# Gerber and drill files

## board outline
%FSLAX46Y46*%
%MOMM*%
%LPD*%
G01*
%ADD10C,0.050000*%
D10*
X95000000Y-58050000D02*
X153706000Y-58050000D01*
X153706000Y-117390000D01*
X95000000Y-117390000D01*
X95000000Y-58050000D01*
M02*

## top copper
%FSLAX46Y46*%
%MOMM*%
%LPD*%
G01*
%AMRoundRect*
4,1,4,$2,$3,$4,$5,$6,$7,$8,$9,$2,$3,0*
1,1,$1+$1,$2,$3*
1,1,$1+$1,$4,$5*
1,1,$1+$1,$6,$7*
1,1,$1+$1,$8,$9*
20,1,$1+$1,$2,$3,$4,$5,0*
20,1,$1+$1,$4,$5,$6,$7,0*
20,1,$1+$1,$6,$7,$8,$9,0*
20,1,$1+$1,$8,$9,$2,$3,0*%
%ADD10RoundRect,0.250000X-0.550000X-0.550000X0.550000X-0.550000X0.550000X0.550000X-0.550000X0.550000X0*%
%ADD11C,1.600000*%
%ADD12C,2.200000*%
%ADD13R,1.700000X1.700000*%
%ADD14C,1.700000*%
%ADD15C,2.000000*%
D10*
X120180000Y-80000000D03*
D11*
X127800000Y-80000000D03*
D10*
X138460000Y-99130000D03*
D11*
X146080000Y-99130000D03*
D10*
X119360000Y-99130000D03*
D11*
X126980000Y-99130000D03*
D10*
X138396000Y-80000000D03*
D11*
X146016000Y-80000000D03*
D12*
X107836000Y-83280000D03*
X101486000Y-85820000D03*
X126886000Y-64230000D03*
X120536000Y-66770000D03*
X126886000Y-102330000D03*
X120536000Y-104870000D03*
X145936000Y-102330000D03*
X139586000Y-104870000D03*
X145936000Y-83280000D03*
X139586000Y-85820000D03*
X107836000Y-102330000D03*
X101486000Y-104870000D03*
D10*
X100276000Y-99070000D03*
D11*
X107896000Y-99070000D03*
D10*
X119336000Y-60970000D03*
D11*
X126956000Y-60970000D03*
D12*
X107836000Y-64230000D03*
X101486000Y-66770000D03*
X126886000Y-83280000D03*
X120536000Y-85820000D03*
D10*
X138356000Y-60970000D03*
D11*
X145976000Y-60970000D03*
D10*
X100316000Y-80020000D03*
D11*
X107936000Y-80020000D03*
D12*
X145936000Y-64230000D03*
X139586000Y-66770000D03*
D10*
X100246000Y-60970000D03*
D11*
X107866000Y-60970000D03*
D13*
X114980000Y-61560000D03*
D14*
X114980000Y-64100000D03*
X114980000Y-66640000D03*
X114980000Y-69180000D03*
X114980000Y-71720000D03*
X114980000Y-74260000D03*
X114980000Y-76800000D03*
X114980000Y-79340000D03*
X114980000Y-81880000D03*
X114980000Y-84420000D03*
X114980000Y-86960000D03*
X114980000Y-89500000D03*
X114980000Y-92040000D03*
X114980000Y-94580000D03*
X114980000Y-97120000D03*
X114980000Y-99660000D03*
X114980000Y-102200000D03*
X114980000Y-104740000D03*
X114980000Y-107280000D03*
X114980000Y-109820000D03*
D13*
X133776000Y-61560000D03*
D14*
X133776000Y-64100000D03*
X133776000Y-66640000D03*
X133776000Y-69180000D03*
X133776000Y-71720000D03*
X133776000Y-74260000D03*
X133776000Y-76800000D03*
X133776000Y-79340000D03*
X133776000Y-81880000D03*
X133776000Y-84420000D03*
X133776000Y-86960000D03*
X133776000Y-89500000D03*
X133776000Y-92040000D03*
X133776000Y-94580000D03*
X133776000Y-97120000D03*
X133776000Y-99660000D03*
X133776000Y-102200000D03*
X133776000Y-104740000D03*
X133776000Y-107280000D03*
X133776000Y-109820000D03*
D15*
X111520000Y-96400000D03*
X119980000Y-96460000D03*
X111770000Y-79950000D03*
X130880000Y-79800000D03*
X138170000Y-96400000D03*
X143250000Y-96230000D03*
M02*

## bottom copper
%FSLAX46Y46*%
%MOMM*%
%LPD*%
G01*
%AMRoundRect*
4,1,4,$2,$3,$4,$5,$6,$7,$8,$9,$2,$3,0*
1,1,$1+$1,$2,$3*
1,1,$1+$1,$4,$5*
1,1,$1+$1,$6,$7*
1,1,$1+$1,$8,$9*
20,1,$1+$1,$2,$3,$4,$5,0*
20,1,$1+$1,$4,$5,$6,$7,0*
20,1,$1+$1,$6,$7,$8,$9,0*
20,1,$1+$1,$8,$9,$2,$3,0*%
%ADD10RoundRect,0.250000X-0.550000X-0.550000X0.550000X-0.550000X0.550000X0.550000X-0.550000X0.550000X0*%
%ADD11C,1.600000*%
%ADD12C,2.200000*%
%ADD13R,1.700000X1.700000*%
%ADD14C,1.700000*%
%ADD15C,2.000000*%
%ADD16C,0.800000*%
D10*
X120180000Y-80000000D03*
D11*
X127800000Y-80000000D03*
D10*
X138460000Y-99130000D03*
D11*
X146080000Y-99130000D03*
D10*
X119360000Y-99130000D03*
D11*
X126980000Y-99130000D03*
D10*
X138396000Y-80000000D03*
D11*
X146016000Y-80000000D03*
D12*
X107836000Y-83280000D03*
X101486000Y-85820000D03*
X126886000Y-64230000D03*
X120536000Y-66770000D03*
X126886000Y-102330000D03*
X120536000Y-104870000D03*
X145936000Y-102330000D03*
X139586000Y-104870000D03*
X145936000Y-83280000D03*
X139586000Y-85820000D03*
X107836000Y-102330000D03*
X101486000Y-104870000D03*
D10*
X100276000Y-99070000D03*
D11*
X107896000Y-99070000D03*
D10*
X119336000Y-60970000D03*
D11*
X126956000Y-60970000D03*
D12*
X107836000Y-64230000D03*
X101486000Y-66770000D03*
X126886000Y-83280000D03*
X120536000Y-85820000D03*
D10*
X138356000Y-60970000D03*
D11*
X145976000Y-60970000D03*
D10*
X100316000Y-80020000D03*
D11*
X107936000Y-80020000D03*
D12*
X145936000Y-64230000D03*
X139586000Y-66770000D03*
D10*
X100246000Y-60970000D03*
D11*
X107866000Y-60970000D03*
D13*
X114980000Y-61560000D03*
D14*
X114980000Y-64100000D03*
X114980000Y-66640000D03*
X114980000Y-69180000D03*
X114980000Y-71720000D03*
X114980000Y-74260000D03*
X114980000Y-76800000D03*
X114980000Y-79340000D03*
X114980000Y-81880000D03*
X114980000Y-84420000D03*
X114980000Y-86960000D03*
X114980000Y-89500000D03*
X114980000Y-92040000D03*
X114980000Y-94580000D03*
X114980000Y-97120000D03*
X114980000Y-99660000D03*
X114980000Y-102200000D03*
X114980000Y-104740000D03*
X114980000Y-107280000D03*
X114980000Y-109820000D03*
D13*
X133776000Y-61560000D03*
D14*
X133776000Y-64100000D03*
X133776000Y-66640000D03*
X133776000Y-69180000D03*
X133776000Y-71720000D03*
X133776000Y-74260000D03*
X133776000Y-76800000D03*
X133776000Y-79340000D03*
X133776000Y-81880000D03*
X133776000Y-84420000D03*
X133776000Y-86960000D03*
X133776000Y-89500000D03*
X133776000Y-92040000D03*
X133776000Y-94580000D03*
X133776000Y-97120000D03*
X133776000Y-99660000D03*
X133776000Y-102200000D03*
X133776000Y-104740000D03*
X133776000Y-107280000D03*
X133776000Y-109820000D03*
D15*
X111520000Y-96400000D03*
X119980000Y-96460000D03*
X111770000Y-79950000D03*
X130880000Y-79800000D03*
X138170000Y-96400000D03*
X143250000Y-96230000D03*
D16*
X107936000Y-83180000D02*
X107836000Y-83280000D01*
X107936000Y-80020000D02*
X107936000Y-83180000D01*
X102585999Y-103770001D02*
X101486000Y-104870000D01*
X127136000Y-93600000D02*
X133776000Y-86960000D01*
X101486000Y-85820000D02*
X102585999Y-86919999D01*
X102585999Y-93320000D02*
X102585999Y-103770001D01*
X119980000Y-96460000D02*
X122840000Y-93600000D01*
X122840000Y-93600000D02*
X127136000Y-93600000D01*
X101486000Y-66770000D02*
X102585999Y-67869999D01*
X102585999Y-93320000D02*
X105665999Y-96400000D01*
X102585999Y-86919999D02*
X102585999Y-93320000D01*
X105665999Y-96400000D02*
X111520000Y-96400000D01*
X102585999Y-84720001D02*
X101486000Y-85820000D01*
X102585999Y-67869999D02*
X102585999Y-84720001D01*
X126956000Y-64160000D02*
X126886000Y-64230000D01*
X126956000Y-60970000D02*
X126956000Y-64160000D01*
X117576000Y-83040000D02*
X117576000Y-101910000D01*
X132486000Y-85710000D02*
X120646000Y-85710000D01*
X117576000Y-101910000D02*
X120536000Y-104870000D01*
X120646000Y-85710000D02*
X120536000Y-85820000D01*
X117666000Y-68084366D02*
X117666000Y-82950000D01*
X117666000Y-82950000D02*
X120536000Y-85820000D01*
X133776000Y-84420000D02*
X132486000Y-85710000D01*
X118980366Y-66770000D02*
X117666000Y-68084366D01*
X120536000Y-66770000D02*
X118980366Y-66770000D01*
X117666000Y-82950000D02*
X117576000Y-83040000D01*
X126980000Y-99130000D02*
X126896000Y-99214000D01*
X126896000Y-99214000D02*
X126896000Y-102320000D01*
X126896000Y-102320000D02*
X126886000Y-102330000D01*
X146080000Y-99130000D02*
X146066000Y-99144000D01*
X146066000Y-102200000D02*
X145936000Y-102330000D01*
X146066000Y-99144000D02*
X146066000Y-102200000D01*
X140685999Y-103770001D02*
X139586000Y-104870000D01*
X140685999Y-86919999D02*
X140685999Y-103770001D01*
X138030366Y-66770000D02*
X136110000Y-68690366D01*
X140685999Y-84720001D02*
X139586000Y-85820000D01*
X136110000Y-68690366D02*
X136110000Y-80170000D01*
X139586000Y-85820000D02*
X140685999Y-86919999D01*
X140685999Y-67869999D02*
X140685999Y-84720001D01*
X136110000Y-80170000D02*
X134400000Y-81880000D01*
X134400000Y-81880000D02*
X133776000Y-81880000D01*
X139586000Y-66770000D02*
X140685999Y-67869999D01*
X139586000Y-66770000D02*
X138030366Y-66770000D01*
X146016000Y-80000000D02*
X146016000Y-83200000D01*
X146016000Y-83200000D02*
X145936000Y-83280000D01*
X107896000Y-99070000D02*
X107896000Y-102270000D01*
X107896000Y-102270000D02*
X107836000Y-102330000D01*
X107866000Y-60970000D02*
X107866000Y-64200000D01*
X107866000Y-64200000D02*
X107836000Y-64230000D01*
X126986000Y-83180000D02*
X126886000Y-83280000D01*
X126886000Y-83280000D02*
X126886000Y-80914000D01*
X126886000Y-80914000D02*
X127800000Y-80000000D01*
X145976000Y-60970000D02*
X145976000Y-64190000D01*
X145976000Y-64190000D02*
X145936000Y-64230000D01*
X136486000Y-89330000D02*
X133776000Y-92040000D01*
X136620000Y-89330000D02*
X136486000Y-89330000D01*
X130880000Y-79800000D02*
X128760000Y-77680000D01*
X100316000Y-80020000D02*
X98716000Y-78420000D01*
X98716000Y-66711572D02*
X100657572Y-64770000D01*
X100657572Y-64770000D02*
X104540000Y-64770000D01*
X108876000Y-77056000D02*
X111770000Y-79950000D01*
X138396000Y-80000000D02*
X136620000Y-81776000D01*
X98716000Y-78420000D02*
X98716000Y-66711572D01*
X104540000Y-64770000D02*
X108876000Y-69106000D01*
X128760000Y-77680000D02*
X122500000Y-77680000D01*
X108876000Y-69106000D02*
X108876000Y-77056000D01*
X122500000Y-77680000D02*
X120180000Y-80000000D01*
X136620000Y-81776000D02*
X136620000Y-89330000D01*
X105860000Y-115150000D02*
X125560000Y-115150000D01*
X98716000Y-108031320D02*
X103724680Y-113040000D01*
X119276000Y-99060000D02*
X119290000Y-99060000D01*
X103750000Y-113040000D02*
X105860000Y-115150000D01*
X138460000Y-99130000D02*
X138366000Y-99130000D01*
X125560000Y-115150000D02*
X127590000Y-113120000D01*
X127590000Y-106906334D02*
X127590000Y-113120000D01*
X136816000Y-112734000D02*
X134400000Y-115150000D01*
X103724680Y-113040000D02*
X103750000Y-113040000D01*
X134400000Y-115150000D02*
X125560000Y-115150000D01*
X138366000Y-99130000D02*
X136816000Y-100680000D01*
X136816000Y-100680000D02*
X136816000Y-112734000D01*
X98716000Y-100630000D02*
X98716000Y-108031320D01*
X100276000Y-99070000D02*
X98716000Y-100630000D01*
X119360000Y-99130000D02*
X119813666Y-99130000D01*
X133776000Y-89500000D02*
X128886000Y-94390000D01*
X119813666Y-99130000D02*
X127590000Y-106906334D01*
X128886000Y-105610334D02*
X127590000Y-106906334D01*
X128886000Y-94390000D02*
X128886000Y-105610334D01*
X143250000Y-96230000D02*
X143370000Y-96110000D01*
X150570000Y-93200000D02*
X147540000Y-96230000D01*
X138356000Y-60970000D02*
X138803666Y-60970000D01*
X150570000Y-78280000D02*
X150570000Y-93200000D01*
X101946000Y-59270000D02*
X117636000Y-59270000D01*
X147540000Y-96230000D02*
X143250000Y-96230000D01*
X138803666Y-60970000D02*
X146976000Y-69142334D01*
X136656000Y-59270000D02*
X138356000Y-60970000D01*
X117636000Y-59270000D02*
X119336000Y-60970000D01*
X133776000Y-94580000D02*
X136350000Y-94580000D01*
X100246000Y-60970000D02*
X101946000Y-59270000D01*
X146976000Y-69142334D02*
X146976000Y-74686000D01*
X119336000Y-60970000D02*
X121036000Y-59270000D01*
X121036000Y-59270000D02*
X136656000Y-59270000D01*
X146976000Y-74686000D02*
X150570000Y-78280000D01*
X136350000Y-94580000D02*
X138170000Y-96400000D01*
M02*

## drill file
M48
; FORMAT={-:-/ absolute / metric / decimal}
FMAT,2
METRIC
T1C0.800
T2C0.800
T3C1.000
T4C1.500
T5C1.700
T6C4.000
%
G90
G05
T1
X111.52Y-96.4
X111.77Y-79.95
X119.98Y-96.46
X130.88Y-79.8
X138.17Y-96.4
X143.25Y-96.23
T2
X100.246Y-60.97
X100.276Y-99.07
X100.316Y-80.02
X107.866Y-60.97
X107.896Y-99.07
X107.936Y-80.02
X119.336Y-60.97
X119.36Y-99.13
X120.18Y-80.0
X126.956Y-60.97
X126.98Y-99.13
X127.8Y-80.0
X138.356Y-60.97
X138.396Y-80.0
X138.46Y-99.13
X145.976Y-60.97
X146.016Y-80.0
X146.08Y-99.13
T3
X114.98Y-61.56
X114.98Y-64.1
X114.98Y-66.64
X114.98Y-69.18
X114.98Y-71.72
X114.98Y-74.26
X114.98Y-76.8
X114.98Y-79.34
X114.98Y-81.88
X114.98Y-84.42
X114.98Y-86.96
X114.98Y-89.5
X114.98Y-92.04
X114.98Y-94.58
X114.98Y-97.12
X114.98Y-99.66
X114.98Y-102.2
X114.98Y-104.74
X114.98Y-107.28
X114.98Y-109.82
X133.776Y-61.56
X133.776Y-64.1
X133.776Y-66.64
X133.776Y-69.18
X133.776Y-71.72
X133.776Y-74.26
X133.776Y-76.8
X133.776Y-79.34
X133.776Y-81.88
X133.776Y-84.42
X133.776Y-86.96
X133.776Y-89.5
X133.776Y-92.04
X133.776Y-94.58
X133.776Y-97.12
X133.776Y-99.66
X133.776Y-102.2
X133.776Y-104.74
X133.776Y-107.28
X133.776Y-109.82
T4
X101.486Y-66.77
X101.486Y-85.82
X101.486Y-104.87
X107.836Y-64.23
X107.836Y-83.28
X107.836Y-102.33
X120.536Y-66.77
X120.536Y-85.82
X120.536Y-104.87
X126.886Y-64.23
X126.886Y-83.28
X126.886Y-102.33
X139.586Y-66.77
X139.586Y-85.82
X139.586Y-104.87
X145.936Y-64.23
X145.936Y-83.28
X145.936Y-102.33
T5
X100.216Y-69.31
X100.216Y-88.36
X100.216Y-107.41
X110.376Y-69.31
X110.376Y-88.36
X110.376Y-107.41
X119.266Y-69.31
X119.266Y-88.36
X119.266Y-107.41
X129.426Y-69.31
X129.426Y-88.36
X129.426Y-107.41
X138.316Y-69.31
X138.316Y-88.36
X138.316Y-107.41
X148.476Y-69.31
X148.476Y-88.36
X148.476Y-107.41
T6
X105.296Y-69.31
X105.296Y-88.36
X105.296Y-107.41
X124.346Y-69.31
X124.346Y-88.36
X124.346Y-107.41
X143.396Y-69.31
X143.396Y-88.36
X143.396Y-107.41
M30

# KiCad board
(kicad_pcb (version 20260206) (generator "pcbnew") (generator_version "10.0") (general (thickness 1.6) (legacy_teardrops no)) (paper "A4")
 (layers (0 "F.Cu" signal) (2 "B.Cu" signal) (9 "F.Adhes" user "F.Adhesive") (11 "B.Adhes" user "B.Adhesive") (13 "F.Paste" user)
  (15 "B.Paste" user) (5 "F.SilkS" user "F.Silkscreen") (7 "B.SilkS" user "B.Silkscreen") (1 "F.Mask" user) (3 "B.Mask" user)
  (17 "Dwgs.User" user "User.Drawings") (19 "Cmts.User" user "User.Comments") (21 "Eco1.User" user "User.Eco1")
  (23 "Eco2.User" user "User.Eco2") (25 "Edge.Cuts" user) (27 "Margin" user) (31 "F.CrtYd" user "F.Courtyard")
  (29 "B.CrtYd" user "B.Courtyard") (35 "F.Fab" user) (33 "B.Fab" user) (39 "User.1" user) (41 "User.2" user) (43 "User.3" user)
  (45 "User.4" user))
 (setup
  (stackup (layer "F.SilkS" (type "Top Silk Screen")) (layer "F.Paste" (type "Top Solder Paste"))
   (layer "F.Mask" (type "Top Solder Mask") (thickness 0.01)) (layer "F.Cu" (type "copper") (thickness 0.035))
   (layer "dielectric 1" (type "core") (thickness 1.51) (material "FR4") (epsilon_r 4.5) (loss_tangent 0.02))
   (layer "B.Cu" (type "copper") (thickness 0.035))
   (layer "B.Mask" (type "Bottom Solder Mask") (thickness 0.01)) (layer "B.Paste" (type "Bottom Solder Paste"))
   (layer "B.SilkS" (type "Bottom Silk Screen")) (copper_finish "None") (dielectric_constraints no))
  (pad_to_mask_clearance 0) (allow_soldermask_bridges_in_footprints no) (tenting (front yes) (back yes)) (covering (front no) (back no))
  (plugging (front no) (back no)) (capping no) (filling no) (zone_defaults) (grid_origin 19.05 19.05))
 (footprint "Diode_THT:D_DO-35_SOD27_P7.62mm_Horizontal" (layer "F.Cu") (at 120.18 80)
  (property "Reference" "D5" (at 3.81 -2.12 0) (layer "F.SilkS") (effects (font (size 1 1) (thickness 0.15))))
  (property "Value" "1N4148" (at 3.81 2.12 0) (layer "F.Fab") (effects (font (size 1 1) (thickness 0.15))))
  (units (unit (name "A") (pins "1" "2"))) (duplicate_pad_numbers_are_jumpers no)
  (pad "1" thru_hole roundrect (at 0 0) (size 1.6 1.6) (drill 0.8) (layers "*.Cu" "*.Mask") (remove_unused_layers no)
   (roundrect_rratio 0.15625) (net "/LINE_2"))
  (pad "2" thru_hole circle (at 7.62 0) (size 1.6 1.6) (drill 0.8) (layers "*.Cu" "*.Mask") (remove_unused_layers no) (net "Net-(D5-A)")))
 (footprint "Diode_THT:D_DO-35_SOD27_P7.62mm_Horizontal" (layer "F.Cu") (at 138.46 99.13)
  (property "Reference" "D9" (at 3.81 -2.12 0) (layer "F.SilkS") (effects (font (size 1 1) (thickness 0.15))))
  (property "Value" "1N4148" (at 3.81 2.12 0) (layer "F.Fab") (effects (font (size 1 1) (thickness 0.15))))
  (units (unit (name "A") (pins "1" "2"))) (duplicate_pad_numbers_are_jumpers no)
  (pad "1" thru_hole roundrect (at 0 0) (size 1.6 1.6) (drill 0.8) (layers "*.Cu" "*.Mask") (remove_unused_layers no)
   (roundrect_rratio 0.15625) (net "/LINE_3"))
  (pad "2" thru_hole circle (at 7.62 0) (size 1.6 1.6) (drill 0.8) (layers "*.Cu" "*.Mask") (remove_unused_layers no) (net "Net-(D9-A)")))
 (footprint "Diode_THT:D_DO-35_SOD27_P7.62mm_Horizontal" (layer "F.Cu") (at 119.36 99.13)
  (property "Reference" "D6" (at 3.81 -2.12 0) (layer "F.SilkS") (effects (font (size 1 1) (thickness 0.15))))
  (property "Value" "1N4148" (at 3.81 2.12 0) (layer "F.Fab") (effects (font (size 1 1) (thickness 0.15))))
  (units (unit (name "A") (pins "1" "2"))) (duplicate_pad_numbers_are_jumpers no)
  (pad "1" thru_hole roundrect (at 0 0) (size 1.6 1.6) (drill 0.8) (layers "*.Cu" "*.Mask") (remove_unused_layers no)
   (roundrect_rratio 0.15625) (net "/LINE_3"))
  (pad "2" thru_hole circle (at 7.62 0) (size 1.6 1.6) (drill 0.8) (layers "*.Cu" "*.Mask") (remove_unused_layers no) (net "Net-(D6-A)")))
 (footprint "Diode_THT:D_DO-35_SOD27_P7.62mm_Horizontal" (layer "F.Cu") (at 138.396 80)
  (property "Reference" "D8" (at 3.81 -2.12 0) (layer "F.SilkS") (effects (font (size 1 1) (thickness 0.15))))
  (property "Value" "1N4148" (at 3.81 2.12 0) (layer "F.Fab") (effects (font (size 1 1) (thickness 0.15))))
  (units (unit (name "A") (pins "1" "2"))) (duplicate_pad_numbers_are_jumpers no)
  (pad "1" thru_hole roundrect (at 0 0) (size 1.6 1.6) (drill 0.8) (layers "*.Cu" "*.Mask") (remove_unused_layers no)
   (roundrect_rratio 0.15625) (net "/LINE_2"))
  (pad "2" thru_hole circle (at 7.62 0) (size 1.6 1.6) (drill 0.8) (layers "*.Cu" "*.Mask") (remove_unused_layers no) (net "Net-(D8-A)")))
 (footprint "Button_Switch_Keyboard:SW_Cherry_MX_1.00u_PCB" (layer "F.Cu") (at 107.836 83.28)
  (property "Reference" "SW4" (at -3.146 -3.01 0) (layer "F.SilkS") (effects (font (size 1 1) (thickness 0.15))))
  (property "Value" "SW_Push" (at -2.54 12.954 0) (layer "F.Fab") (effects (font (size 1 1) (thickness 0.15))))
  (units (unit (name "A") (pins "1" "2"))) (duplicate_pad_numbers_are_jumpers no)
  (pad "" np_thru_hole circle (at -7.62 5.08) (size 1.7 1.7) (drill 1.7) (layers "*.Cu" "*.Mask"))
  (pad "" np_thru_hole circle (at -2.54 5.08) (size 4 4) (drill 4) (layers "*.Cu" "*.Mask"))
  (pad "" np_thru_hole circle (at 2.54 5.08) (size 1.7 1.7) (drill 1.7) (layers "*.Cu" "*.Mask"))
  (pad "1" thru_hole circle (at 0 0) (size 2.2 2.2) (drill 1.5) (layers "*.Cu" "*.Mask") (remove_unused_layers no) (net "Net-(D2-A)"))
  (pad "2" thru_hole circle (at -6.35 2.54) (size 2.2 2.2) (drill 1.5) (layers "*.Cu" "*.Mask") (remove_unused_layers no) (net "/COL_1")))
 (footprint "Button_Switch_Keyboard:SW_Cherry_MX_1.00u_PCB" (layer "F.Cu") (at 126.886 64.23)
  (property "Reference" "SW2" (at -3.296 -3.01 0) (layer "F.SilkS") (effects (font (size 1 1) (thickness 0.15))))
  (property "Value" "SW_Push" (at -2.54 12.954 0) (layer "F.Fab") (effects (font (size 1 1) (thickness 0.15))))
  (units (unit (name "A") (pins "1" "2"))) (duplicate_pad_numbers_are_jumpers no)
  (pad "" np_thru_hole circle (at -7.62 5.08) (size 1.7 1.7) (drill 1.7) (layers "*.Cu" "*.Mask"))
  (pad "" np_thru_hole circle (at -2.54 5.08) (size 4 4) (drill 4) (layers "*.Cu" "*.Mask"))
  (pad "" np_thru_hole circle (at 2.54 5.08) (size 1.7 1.7) (drill 1.7) (layers "*.Cu" "*.Mask"))
  (pad "1" thru_hole circle (at 0 0) (size 2.2 2.2) (drill 1.5) (layers "*.Cu" "*.Mask") (remove_unused_layers no) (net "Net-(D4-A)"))
  (pad "2" thru_hole circle (at -6.35 2.54) (size 2.2 2.2) (drill 1.5) (layers "*.Cu" "*.Mask") (remove_unused_layers no) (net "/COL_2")))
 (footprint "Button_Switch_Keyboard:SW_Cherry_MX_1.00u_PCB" (layer "F.Cu") (at 126.886 102.33)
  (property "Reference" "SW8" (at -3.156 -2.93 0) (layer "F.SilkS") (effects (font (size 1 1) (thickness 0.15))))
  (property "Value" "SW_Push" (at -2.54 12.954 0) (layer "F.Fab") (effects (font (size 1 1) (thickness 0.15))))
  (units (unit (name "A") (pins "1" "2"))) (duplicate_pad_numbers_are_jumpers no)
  (pad "" np_thru_hole circle (at -7.62 5.08) (size 1.7 1.7) (drill 1.7) (layers "*.Cu" "*.Mask"))
  (pad "" np_thru_hole circle (at -2.54 5.08) (size 4 4) (drill 4) (layers "*.Cu" "*.Mask"))
  (pad "" np_thru_hole circle (at 2.54 5.08) (size 1.7 1.7) (drill 1.7) (layers "*.Cu" "*.Mask"))
  (pad "1" thru_hole circle (at 0 0) (size 2.2 2.2) (drill 1.5) (layers "*.Cu" "*.Mask") (remove_unused_layers no) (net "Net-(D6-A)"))
  (pad "2" thru_hole circle (at -6.35 2.54) (size 2.2 2.2) (drill 1.5) (layers "*.Cu" "*.Mask") (remove_unused_layers no) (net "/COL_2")))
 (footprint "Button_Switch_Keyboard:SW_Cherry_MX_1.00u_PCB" (layer "F.Cu") (at 145.936 102.33)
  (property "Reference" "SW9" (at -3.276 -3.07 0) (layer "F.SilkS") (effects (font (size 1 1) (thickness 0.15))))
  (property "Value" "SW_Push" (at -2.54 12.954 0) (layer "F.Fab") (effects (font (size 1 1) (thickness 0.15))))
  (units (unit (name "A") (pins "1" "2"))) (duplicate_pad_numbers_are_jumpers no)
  (pad "" np_thru_hole circle (at -7.62 5.08) (size 1.7 1.7) (drill 1.7) (layers "*.Cu" "*.Mask"))
  (pad "" np_thru_hole circle (at -2.54 5.08) (size 4 4) (drill 4) (layers "*.Cu" "*.Mask"))
  (pad "" np_thru_hole circle (at 2.54 5.08) (size 1.7 1.7) (drill 1.7) (layers "*.Cu" "*.Mask"))
  (pad "1" thru_hole circle (at 0 0) (size 2.2 2.2) (drill 1.5) (layers "*.Cu" "*.Mask") (remove_unused_layers no) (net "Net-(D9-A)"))
  (pad "2" thru_hole circle (at -6.35 2.54) (size 2.2 2.2) (drill 1.5) (layers "*.Cu" "*.Mask") (remove_unused_layers no) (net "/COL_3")))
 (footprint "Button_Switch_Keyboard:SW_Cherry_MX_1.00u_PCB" (layer "F.Cu") (at 145.936 83.28)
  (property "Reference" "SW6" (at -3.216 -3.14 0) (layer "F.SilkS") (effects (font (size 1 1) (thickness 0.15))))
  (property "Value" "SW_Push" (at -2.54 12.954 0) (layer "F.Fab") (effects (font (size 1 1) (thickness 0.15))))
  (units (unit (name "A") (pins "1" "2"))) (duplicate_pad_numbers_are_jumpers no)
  (pad "" np_thru_hole circle (at -7.62 5.08) (size 1.7 1.7) (drill 1.7) (layers "*.Cu" "*.Mask"))
  (pad "" np_thru_hole circle (at -2.54 5.08) (size 4 4) (drill 4) (layers "*.Cu" "*.Mask"))
  (pad "" np_thru_hole circle (at 2.54 5.08) (size 1.7 1.7) (drill 1.7) (layers "*.Cu" "*.Mask"))
  (pad "1" thru_hole circle (at 0 0) (size 2.2 2.2) (drill 1.5) (layers "*.Cu" "*.Mask") (remove_unused_layers no) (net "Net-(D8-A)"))
  (pad "2" thru_hole circle (at -6.35 2.54) (size 2.2 2.2) (drill 1.5) (layers "*.Cu" "*.Mask") (remove_unused_layers no) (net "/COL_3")))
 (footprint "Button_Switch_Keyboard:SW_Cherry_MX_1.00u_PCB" (layer "F.Cu") (at 107.836 102.33)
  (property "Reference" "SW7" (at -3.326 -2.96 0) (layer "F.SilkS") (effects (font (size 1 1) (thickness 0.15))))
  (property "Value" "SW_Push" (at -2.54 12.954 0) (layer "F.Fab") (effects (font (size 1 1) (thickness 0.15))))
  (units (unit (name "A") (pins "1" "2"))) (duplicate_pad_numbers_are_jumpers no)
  (pad "" np_thru_hole circle (at -7.62 5.08) (size 1.7 1.7) (drill 1.7) (layers "*.Cu" "*.Mask"))
  (pad "" np_thru_hole circle (at -2.54 5.08) (size 4 4) (drill 4) (layers "*.Cu" "*.Mask"))
  (pad "" np_thru_hole circle (at 2.54 5.08) (size 1.7 1.7) (drill 1.7) (layers "*.Cu" "*.Mask"))
  (pad "1" thru_hole circle (at 0 0) (size 2.2 2.2) (drill 1.5) (layers "*.Cu" "*.Mask") (remove_unused_layers no) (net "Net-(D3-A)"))
  (pad "2" thru_hole circle (at -6.35 2.54) (size 2.2 2.2) (drill 1.5) (layers "*.Cu" "*.Mask") (remove_unused_layers no) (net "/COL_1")))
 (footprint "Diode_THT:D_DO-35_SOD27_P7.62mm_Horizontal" (layer "F.Cu") (at 100.276 99.07)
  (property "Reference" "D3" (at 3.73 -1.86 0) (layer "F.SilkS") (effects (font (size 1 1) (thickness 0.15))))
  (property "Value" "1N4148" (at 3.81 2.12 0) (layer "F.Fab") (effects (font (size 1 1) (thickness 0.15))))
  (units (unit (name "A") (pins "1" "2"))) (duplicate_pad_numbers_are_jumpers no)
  (pad "1" thru_hole roundrect (at 0 0) (size 1.6 1.6) (drill 0.8) (layers "*.Cu" "*.Mask") (remove_unused_layers no)
   (roundrect_rratio 0.15625) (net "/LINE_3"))
  (pad "2" thru_hole circle (at 7.62 0) (size 1.6 1.6) (drill 0.8) (layers "*.Cu" "*.Mask") (remove_unused_layers no) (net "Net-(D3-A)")))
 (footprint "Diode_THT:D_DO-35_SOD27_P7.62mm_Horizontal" (layer "F.Cu") (at 119.336 60.97)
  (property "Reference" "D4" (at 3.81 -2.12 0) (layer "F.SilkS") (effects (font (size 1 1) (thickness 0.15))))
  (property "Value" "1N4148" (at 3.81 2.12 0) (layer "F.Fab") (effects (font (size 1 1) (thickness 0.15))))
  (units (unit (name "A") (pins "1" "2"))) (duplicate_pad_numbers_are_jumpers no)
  (pad "1" thru_hole roundrect (at 0 0) (size 1.6 1.6) (drill 0.8) (layers "*.Cu" "*.Mask") (remove_unused_layers no)
   (roundrect_rratio 0.15625) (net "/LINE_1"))
  (pad "2" thru_hole circle (at 7.62 0) (size 1.6 1.6) (drill 0.8) (layers "*.Cu" "*.Mask") (remove_unused_layers no) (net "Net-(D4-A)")))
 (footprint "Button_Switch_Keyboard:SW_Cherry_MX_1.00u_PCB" (layer "F.Cu") (at 107.836 64.23)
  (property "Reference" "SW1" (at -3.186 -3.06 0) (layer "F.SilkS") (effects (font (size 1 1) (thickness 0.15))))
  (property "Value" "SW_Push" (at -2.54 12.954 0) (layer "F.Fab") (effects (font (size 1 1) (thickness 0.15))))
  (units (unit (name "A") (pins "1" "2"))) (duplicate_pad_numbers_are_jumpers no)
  (pad "" np_thru_hole circle (at -7.62 5.08) (size 1.7 1.7) (drill 1.7) (layers "*.Cu" "*.Mask"))
  (pad "" np_thru_hole circle (at -2.54 5.08) (size 4 4) (drill 4) (layers "*.Cu" "*.Mask"))
  (pad "" np_thru_hole circle (at 2.54 5.08) (size 1.7 1.7) (drill 1.7) (layers "*.Cu" "*.Mask"))
  (pad "1" thru_hole circle (at 0 0) (size 2.2 2.2) (drill 1.5) (layers "*.Cu" "*.Mask") (remove_unused_layers no) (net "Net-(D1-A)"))
  (pad "2" thru_hole circle (at -6.35 2.54) (size 2.2 2.2) (drill 1.5) (layers "*.Cu" "*.Mask") (remove_unused_layers no) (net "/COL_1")))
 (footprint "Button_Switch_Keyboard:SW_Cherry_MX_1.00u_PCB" (layer "F.Cu") (at 126.886 83.28)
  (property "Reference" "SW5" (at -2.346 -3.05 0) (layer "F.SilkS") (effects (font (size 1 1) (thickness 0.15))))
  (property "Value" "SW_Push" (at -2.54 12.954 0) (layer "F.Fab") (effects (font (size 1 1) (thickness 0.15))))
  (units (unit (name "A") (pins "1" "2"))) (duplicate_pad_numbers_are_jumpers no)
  (pad "" np_thru_hole circle (at -7.62 5.08) (size 1.7 1.7) (drill 1.7) (layers "*.Cu" "*.Mask"))
  (pad "" np_thru_hole circle (at -2.54 5.08) (size 4 4) (drill 4) (layers "*.Cu" "*.Mask"))
  (pad "" np_thru_hole circle (at 2.54 5.08) (size 1.7 1.7) (drill 1.7) (layers "*.Cu" "*.Mask"))
  (pad "1" thru_hole circle (at 0 0) (size 2.2 2.2) (drill 1.5) (layers "*.Cu" "*.Mask") (remove_unused_layers no) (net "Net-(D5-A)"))
  (pad "2" thru_hole circle (at -6.35 2.54) (size 2.2 2.2) (drill 1.5) (layers "*.Cu" "*.Mask") (remove_unused_layers no) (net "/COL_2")))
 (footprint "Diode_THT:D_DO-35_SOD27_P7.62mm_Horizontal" (layer "F.Cu") (at 138.356 60.97)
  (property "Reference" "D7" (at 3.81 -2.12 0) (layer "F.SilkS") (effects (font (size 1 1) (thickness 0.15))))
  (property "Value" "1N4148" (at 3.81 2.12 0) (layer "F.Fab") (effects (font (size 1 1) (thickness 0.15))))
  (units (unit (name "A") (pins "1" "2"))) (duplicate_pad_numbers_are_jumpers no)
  (pad "1" thru_hole roundrect (at 0 0) (size 1.6 1.6) (drill 0.8) (layers "*.Cu" "*.Mask") (remove_unused_layers no)
   (roundrect_rratio 0.15625) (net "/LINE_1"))
  (pad "2" thru_hole circle (at 7.62 0) (size 1.6 1.6) (drill 0.8) (layers "*.Cu" "*.Mask") (remove_unused_layers no) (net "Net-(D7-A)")))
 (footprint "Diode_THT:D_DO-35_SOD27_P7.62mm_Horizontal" (layer "F.Cu") (at 100.316 80.02)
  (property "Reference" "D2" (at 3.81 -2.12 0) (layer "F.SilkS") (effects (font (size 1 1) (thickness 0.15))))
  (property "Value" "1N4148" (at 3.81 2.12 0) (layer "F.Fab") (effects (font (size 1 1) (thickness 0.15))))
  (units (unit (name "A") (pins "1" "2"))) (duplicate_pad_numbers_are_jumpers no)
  (pad "1" thru_hole roundrect (at 0 0) (size 1.6 1.6) (drill 0.8) (layers "*.Cu" "*.Mask") (remove_unused_layers no)
   (roundrect_rratio 0.15625) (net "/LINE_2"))
  (pad "2" thru_hole circle (at 7.62 0) (size 1.6 1.6) (drill 0.8) (layers "*.Cu" "*.Mask") (remove_unused_layers no) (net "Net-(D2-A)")))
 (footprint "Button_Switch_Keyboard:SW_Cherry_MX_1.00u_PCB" (layer "F.Cu") (at 145.936 64.23)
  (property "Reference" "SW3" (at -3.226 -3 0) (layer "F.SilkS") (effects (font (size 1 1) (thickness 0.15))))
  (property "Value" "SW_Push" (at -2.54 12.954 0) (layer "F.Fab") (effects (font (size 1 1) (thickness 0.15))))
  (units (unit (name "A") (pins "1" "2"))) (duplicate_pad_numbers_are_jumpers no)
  (pad "" np_thru_hole circle (at -7.62 5.08) (size 1.7 1.7) (drill 1.7) (layers "*.Cu" "*.Mask"))
  (pad "" np_thru_hole circle (at -2.54 5.08) (size 4 4) (drill 4) (layers "*.Cu" "*.Mask"))
  (pad "" np_thru_hole circle (at 2.54 5.08) (size 1.7 1.7) (drill 1.7) (layers "*.Cu" "*.Mask"))
  (pad "1" thru_hole circle (at 0 0) (size 2.2 2.2) (drill 1.5) (layers "*.Cu" "*.Mask") (remove_unused_layers no) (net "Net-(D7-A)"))
  (pad "2" thru_hole circle (at -6.35 2.54) (size 2.2 2.2) (drill 1.5) (layers "*.Cu" "*.Mask") (remove_unused_layers no) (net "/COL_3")))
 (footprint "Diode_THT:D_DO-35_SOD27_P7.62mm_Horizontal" (layer "F.Cu") (at 100.246 60.97)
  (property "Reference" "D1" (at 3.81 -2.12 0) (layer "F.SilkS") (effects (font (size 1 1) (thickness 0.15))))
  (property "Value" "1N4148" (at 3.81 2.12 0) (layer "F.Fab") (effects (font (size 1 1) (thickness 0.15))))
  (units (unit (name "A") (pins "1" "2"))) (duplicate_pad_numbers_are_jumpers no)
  (pad "1" thru_hole roundrect (at 0 0) (size 1.6 1.6) (drill 0.8) (layers "*.Cu" "*.Mask") (remove_unused_layers no)
   (roundrect_rratio 0.15625) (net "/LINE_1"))
  (pad "2" thru_hole circle (at 7.62 0) (size 1.6 1.6) (drill 0.8) (layers "*.Cu" "*.Mask") (remove_unused_layers no) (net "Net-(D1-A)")))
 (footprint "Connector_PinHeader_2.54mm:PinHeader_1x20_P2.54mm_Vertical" (layer "B.Cu") (at 114.98 61.56 180)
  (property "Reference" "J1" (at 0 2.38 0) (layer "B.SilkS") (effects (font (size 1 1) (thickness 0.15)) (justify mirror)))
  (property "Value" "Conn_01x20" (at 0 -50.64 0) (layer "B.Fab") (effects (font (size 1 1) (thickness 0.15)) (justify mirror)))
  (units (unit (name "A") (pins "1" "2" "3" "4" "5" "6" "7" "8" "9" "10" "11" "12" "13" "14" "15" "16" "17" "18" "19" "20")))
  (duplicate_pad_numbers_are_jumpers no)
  (pad "1" thru_hole rect (at 0 0 180) (size 1.7 1.7) (drill 1) (layers "*.Cu" "*.Mask") (remove_unused_layers no)
   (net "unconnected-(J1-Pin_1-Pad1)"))
  (pad "2" thru_hole circle (at 0 -2.54 180) (size 1.7 1.7) (drill 1) (layers "*.Cu" "*.Mask") (remove_unused_layers no)
   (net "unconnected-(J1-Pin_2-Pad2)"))
  (pad "3" thru_hole circle (at 0 -5.08 180) (size 1.7 1.7) (drill 1) (layers "*.Cu" "*.Mask") (remove_unused_layers no)
   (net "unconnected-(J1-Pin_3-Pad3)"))
  (pad "4" thru_hole circle (at 0 -7.62 180) (size 1.7 1.7) (drill 1) (layers "*.Cu" "*.Mask") (remove_unused_layers no)
   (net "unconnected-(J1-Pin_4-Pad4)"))
  (pad "5" thru_hole circle (at 0 -10.16 180) (size 1.7 1.7) (drill 1) (layers "*.Cu" "*.Mask") (remove_unused_layers no)
   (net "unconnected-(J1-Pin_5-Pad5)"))
  (pad "6" thru_hole circle (at 0 -12.7 180) (size 1.7 1.7) (drill 1) (layers "*.Cu" "*.Mask") (remove_unused_layers no)
   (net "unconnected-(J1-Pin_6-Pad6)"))
  (pad "7" thru_hole circle (at 0 -15.24 180) (size 1.7 1.7) (drill 1) (layers "*.Cu" "*.Mask") (remove_unused_layers no)
   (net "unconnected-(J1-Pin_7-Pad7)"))
  (pad "8" thru_hole circle (at 0 -17.78 180) (size 1.7 1.7) (drill 1) (layers "*.Cu" "*.Mask") (remove_unused_layers no)
   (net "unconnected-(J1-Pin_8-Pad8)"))
  (pad "9" thru_hole circle (at 0 -20.32 180) (size 1.7 1.7) (drill 1) (layers "*.Cu" "*.Mask") (remove_unused_layers no)
   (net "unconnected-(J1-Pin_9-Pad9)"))
  (pad "10" thru_hole circle (at 0 -22.86 180) (size 1.7 1.7) (drill 1) (layers "*.Cu" "*.Mask") (remove_unused_layers no)
   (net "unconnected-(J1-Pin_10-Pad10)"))
  (pad "11" thru_hole circle (at 0 -25.4 180) (size 1.7 1.7) (drill 1) (layers "*.Cu" "*.Mask") (remove_unused_layers no)
   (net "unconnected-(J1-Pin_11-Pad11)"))
  (pad "12" thru_hole circle (at 0 -27.94 180) (size 1.7 1.7) (drill 1) (layers "*.Cu" "*.Mask") (remove_unused_layers no)
   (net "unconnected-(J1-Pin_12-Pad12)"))
  (pad "13" thru_hole circle (at 0 -30.48 180) (size 1.7 1.7) (drill 1) (layers "*.Cu" "*.Mask") (remove_unused_layers no)
   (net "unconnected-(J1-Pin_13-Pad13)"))
  (pad "14" thru_hole circle (at 0 -33.02 180) (size 1.7 1.7) (drill 1) (layers "*.Cu" "*.Mask") (remove_unused_layers no)
   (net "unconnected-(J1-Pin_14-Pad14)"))
  (pad "15" thru_hole circle (at 0 -35.56 180) (size 1.7 1.7) (drill 1) (layers "*.Cu" "*.Mask") (remove_unused_layers no)
   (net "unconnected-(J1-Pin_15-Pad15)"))
  (pad "16" thru_hole circle (at 0 -38.1 180) (size 1.7 1.7) (drill 1) (layers "*.Cu" "*.Mask") (remove_unused_layers no)
   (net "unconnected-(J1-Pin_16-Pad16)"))
  (pad "17" thru_hole circle (at 0 -40.64 180) (size 1.7 1.7) (drill 1) (layers "*.Cu" "*.Mask") (remove_unused_layers no)
   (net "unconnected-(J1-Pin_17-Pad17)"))
  (pad "18" thru_hole circle (at 0 -43.18 180) (size 1.7 1.7) (drill 1) (layers "*.Cu" "*.Mask") (remove_unused_layers no)
   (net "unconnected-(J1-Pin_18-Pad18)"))
  (pad "19" thru_hole circle (at 0 -45.72 180) (size 1.7 1.7) (drill 1) (layers "*.Cu" "*.Mask") (remove_unused_layers no)
   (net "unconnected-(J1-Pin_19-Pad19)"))
  (pad "20" thru_hole circle (at 0 -48.26 180) (size 1.7 1.7) (drill 1) (layers "*.Cu" "*.Mask") (remove_unused_layers no)
   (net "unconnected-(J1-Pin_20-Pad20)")))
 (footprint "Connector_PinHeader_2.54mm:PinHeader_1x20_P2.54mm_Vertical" (layer "B.Cu") (at 133.776 61.56 180)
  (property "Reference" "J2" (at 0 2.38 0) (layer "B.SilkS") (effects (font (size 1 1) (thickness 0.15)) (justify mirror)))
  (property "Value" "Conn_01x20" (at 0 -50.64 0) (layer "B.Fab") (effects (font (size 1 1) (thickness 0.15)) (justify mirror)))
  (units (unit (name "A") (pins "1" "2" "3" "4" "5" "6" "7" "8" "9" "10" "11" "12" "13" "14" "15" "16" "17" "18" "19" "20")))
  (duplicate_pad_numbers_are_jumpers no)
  (pad "1" thru_hole rect (at 0 0 180) (size 1.7 1.7) (drill 1) (layers "*.Cu" "*.Mask") (remove_unused_layers no)
   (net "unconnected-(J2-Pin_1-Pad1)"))
  (pad "2" thru_hole circle (at 0 -2.54 180) (size 1.7 1.7) (drill 1) (layers "*.Cu" "*.Mask") (remove_unused_layers no)
   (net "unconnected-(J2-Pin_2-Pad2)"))
  (pad "3" thru_hole circle (at 0 -5.08 180) (size 1.7 1.7) (drill 1) (layers "*.Cu" "*.Mask") (remove_unused_layers no)
   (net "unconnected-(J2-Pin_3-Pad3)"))
  (pad "4" thru_hole circle (at 0 -7.62 180) (size 1.7 1.7) (drill 1) (layers "*.Cu" "*.Mask") (remove_unused_layers no)
   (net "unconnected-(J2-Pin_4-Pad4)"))
  (pad "5" thru_hole circle (at 0 -10.16 180) (size 1.7 1.7) (drill 1) (layers "*.Cu" "*.Mask") (remove_unused_layers no)
   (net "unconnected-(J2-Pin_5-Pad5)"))
  (pad "6" thru_hole circle (at 0 -12.7 180) (size 1.7 1.7) (drill 1) (layers "*.Cu" "*.Mask") (remove_unused_layers no)
   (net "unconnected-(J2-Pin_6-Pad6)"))
  (pad "7" thru_hole circle (at 0 -15.24 180) (size 1.7 1.7) (drill 1) (layers "*.Cu" "*.Mask") (remove_unused_layers no)
   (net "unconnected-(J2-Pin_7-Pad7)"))
  (pad "8" thru_hole circle (at 0 -17.78 180) (size 1.7 1.7) (drill 1) (layers "*.Cu" "*.Mask") (remove_unused_layers no)
   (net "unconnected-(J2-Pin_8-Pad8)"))
  (pad "9" thru_hole circle (at 0 -20.32 180) (size 1.7 1.7) (drill 1) (layers "*.Cu" "*.Mask") (remove_unused_layers no) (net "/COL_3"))
  (pad "10" thru_hole circle (at 0 -22.86 180) (size 1.7 1.7) (drill 1) (layers "*.Cu" "*.Mask") (remove_unused_layers no) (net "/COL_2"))
  (pad "11" thru_hole circle (at 0 -25.4 180) (size 1.7 1.7) (drill 1) (layers "*.Cu" "*.Mask") (remove_unused_layers no) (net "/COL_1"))
  (pad "12" thru_hole circle (at 0 -27.94 180) (size 1.7 1.7) (drill 1) (layers "*.Cu" "*.Mask") (remove_unused_layers no) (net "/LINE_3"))
  (pad "13" thru_hole circle (at 0 -30.48 180) (size 1.7 1.7) (drill 1) (layers "*.Cu" "*.Mask") (remove_unused_layers no) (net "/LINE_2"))
  (pad "14" thru_hole circle (at 0 -33.02 180) (size 1.7 1.7) (drill 1) (layers "*.Cu" "*.Mask") (remove_unused_layers no) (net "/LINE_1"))
  (pad "15" thru_hole circle (at 0 -35.56 180) (size 1.7 1.7) (drill 1) (layers "*.Cu" "*.Mask") (remove_unused_layers no)
   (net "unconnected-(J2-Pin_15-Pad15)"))
  (pad "16" thru_hole circle (at 0 -38.1 180) (size 1.7 1.7) (drill 1) (layers "*.Cu" "*.Mask") (remove_unused_layers no)
   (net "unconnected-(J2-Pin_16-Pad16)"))
  (pad "17" thru_hole circle (at 0 -40.64 180) (size 1.7 1.7) (drill 1) (layers "*.Cu" "*.Mask") (remove_unused_layers no)
   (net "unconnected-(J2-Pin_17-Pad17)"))
  (pad "18" thru_hole circle (at 0 -43.18 180) (size 1.7 1.7) (drill 1) (layers "*.Cu" "*.Mask") (remove_unused_layers no)
   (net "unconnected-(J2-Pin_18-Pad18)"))
  (pad "19" thru_hole circle (at 0 -45.72 180) (size 1.7 1.7) (drill 1) (layers "*.Cu" "*.Mask") (remove_unused_layers no)
   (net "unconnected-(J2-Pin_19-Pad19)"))
  (pad "20" thru_hole circle (at 0 -48.26 180) (size 1.7 1.7) (drill 1) (layers "*.Cu" "*.Mask") (remove_unused_layers no)
   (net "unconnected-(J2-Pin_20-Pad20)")))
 (gr_rect (start 95 58.05) (end 153.706 117.39) (stroke (width 0.05) (type default)) (fill no) (layer "Edge.Cuts"))
 (segment (start 107.936 83.18) (end 107.836 83.28) (width 0.8) (layer "B.Cu") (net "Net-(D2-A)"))
 (segment (start 107.936 80.02) (end 107.936 83.18) (width 0.8) (layer "B.Cu") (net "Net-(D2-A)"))
 (via (at 111.52 96.4) (size 2) (drill 0.8) (layers "F.Cu" "B.Cu") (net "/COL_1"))
 (via (at 119.98 96.46) (size 2) (drill 0.8) (layers "F.Cu" "B.Cu") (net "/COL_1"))
 (segment (start 102.585999 103.770001) (end 101.486 104.87) (width 0.8) (layer "B.Cu") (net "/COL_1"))
 (segment (start 127.136 93.6) (end 133.776 86.96) (width 0.8) (layer "B.Cu") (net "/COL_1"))
 (segment (start 101.486 85.82) (end 102.585999 86.919999) (width 0.8) (layer "B.Cu") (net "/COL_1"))
 (segment (start 102.585999 93.32) (end 102.585999 103.770001) (width 0.8) (layer "B.Cu") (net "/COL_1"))
 (segment (start 119.98 96.46) (end 122.84 93.6) (width 0.8) (layer "B.Cu") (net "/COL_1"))
 (segment (start 122.84 93.6) (end 127.136 93.6) (width 0.8) (layer "B.Cu") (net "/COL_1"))
 (segment (start 101.486 66.77) (end 102.585999 67.869999) (width 0.8) (layer "B.Cu") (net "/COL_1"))
 (segment (start 102.585999 93.32) (end 105.665999 96.4) (width 0.8) (layer "B.Cu") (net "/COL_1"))
 (segment (start 102.585999 86.919999) (end 102.585999 93.32) (width 0.8) (layer "B.Cu") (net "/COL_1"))
 (segment (start 105.665999 96.4) (end 111.52 96.4) (width 0.8) (layer "B.Cu") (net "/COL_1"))
 (segment (start 102.585999 84.720001) (end 101.486 85.82) (width 0.8) (layer "B.Cu") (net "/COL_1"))
 (segment (start 102.585999 67.869999) (end 102.585999 84.720001) (width 0.8) (layer "B.Cu") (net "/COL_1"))
 (segment (start 126.956 64.16) (end 126.886 64.23) (width 0.8) (layer "B.Cu") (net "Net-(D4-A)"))
 (segment (start 126.956 60.97) (end 126.956 64.16) (width 0.8) (layer "B.Cu") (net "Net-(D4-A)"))
 (segment (start 117.576 83.04) (end 117.576 101.91) (width 0.8) (layer "B.Cu") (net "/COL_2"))
 (segment (start 132.486 85.71) (end 120.646 85.71) (width 0.8) (layer "B.Cu") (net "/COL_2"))
 (segment (start 117.576 101.91) (end 120.536 104.87) (width 0.8) (layer "B.Cu") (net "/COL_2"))
 (segment (start 120.646 85.71) (end 120.536 85.82) (width 0.8) (layer "B.Cu") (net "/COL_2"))
 (segment (start 117.666 68.084366) (end 117.666 82.95) (width 0.8) (layer "B.Cu") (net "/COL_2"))
 (segment (start 117.666 82.95) (end 120.536 85.82) (width 0.8) (layer "B.Cu") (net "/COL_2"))
 (segment (start 133.776 84.42) (end 132.486 85.71) (width 0.8) (layer "B.Cu") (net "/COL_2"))
 (segment (start 118.980366 66.77) (end 117.666 68.084366) (width 0.8) (layer "B.Cu") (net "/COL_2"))
 (segment (start 120.536 66.77) (end 118.980366 66.77) (width 0.8) (layer "B.Cu") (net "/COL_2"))
 (segment (start 117.666 82.95) (end 117.576 83.04) (width 0.8) (layer "B.Cu") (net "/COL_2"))
 (segment (start 126.98 99.13) (end 126.896 99.214) (width 0.8) (layer "B.Cu") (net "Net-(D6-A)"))
 (segment (start 126.896 99.214) (end 126.896 102.32) (width 0.8) (layer "B.Cu") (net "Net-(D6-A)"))
 (segment (start 126.896 102.32) (end 126.886 102.33) (width 0.8) (layer "B.Cu") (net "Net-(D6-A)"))
 (segment (start 146.08 99.13) (end 146.066 99.144) (width 0.8) (layer "B.Cu") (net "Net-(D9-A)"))
 (segment (start 146.066 102.2) (end 145.936 102.33) (width 0.8) (layer "B.Cu") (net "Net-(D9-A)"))
 (segment (start 146.066 99.144) (end 146.066 102.2) (width 0.8) (layer "B.Cu") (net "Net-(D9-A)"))
 (segment (start 140.685999 103.770001) (end 139.586 104.87) (width 0.8) (layer "B.Cu") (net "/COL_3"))
 (segment (start 140.685999 86.919999) (end 140.685999 103.770001) (width 0.8) (layer "B.Cu") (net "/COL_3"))
 (segment (start 138.030366 66.77) (end 136.11 68.690366) (width 0.8) (layer "B.Cu") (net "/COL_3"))
 (segment (start 140.685999 84.720001) (end 139.586 85.82) (width 0.8) (layer "B.Cu") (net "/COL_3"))
 (segment (start 136.11 68.690366) (end 136.11 80.17) (width 0.8) (layer "B.Cu") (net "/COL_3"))
 (segment (start 139.586 85.82) (end 140.685999 86.919999) (width 0.8) (layer "B.Cu") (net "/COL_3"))
 (segment (start 140.685999 67.869999) (end 140.685999 84.720001) (width 0.8) (layer "B.Cu") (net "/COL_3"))
 (segment (start 136.11 80.17) (end 134.4 81.88) (width 0.8) (layer "B.Cu") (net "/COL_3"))
 (segment (start 134.4 81.88) (end 133.776 81.88) (width 0.8) (layer "B.Cu") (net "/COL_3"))
 (segment (start 139.586 66.77) (end 140.685999 67.869999) (width 0.8) (layer "B.Cu") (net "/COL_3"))
 (segment (start 139.586 66.77) (end 138.030366 66.77) (width 0.8) (layer "B.Cu") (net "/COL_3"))
 (segment (start 146.016 80) (end 146.016 83.2) (width 0.8) (layer "B.Cu") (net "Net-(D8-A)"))
 (segment (start 146.016 83.2) (end 145.936 83.28) (width 0.8) (layer "B.Cu") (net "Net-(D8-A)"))
 (segment (start 107.896 99.07) (end 107.896 102.27) (width 0.8) (layer "B.Cu") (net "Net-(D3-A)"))
 (segment (start 107.896 102.27) (end 107.836 102.33) (width 0.8) (layer "B.Cu") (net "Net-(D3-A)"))
 (segment (start 107.866 60.97) (end 107.866 64.2) (width 0.8) (layer "B.Cu") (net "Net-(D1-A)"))
 (segment (start 107.866 64.2) (end 107.836 64.23) (width 0.8) (layer "B.Cu") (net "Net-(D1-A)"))
 (segment (start 126.986 83.18) (end 126.886 83.28) (width 0.8) (layer "B.Cu") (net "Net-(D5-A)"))
 (segment (start 126.886 83.28) (end 126.886 80.914) (width 0.8) (layer "B.Cu") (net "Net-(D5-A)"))
 (segment (start 126.886 80.914) (end 127.8 80) (width 0.8) (layer "B.Cu") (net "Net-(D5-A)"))
 (segment (start 145.976 60.97) (end 145.976 64.19) (width 0.8) (layer "B.Cu") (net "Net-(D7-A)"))
 (segment (start 145.976 64.19) (end 145.936 64.23) (width 0.8) (layer "B.Cu") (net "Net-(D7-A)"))
 (via (at 111.77 79.95) (size 2) (drill 0.8) (layers "F.Cu" "B.Cu") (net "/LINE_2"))
 (via (at 130.88 79.8) (size 2) (drill 0.8) (layers "F.Cu" "B.Cu") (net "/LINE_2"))
 (segment (start 136.486 89.33) (end 133.776 92.04) (width 0.8) (layer "B.Cu") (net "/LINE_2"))
 (segment (start 136.62 89.33) (end 136.486 89.33) (width 0.8) (layer "B.Cu") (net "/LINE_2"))
 (segment (start 130.88 79.8) (end 128.76 77.68) (width 0.8) (layer "B.Cu") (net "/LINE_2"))
 (segment (start 100.316 80.02) (end 98.716 78.42) (width 0.8) (layer "B.Cu") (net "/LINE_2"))
 (segment (start 98.716 66.711572) (end 100.657572 64.77) (width 0.8) (layer "B.Cu") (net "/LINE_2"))
 (segment (start 100.657572 64.77) (end 104.54 64.77) (width 0.8) (layer "B.Cu") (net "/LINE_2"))
 (segment (start 108.876 77.056) (end 111.77 79.95) (width 0.8) (layer "B.Cu") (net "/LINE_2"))
 (segment (start 138.396 80) (end 136.62 81.776) (width 0.8) (layer "B.Cu") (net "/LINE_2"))
 (segment (start 98.716 78.42) (end 98.716 66.711572) (width 0.8) (layer "B.Cu") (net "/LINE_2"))
 (segment (start 104.54 64.77) (end 108.876 69.106) (width 0.8) (layer "B.Cu") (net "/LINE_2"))
 (segment (start 128.76 77.68) (end 122.5 77.68) (width 0.8) (layer "B.Cu") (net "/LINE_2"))
 (segment (start 108.876 69.106) (end 108.876 77.056) (width 0.8) (layer "B.Cu") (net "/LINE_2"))
 (segment (start 122.5 77.68) (end 120.18 80) (width 0.8) (layer "B.Cu") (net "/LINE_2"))
 (segment (start 136.62 81.776) (end 136.62 89.33) (width 0.8) (layer "B.Cu") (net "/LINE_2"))
 (segment (start 105.86 115.15) (end 125.56 115.15) (width 0.8) (layer "B.Cu") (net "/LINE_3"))
 (segment (start 98.716 108.03132) (end 103.72468 113.04) (width 0.8) (layer "B.Cu") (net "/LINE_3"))
 (segment (start 119.276 99.06) (end 119.29 99.06) (width 0.8) (layer "B.Cu") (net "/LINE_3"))
 (segment (start 103.75 113.04) (end 105.86 115.15) (width 0.8) (layer "B.Cu") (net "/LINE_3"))
 (segment (start 138.46 99.13) (end 138.366 99.13) (width 0.8) (layer "B.Cu") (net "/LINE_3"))
 (segment (start 125.56 115.15) (end 127.59 113.12) (width 0.8) (layer "B.Cu") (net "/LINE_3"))
 (segment (start 127.59 106.906334) (end 127.59 113.12) (width 0.8) (layer "B.Cu") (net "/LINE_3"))
 (segment (start 136.816 112.734) (end 134.4 115.15) (width 0.8) (layer "B.Cu") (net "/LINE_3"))
 (segment (start 103.72468 113.04) (end 103.75 113.04) (width 0.8) (layer "B.Cu") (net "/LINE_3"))
 (segment (start 134.4 115.15) (end 125.56 115.15) (width 0.8) (layer "B.Cu") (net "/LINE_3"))
 (segment (start 138.366 99.13) (end 136.816 100.68) (width 0.8) (layer "B.Cu") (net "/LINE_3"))
 (segment (start 136.816 100.68) (end 136.816 112.734) (width 0.8) (layer "B.Cu") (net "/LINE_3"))
 (segment (start 98.716 100.63) (end 98.716 108.03132) (width 0.8) (layer "B.Cu") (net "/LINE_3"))
 (segment (start 100.276 99.07) (end 98.716 100.63) (width 0.8) (layer "B.Cu") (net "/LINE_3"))
 (segment (start 119.36 99.13) (end 119.813666 99.13) (width 0.8) (layer "B.Cu") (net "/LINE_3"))
 (segment (start 133.776 89.5) (end 128.886 94.39) (width 0.8) (layer "B.Cu") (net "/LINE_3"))
 (segment (start 119.813666 99.13) (end 127.59 106.906334) (width 0.8) (layer "B.Cu") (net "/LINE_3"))
 (segment (start 128.886 105.610334) (end 127.59 106.906334) (width 0.8) (layer "B.Cu") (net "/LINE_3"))
 (segment (start 128.886 94.39) (end 128.886 105.610334) (width 0.8) (layer "B.Cu") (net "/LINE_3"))
 (via (at 138.17 96.4) (size 2) (drill 0.8) (layers "F.Cu" "B.Cu") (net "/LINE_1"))
 (via (at 143.25 96.23) (size 2) (drill 0.8) (layers "F.Cu" "B.Cu") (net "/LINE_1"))
 (segment (start 143.25 96.23) (end 143.37 96.11) (width 0.8) (layer "B.Cu") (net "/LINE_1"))
 (segment (start 150.57 93.2) (end 147.54 96.23) (width 0.8) (layer "B.Cu") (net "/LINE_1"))
 (segment (start 138.356 60.97) (end 138.803666 60.97) (width 0.8) (layer "B.Cu") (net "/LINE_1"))
 (segment (start 150.57 78.28) (end 150.57 93.2) (width 0.8) (layer "B.Cu") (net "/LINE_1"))
 (segment (start 101.946 59.27) (end 117.636 59.27) (width 0.8) (layer "B.Cu") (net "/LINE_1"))
 (segment (start 147.54 96.23) (end 143.25 96.23) (width 0.8) (layer "B.Cu") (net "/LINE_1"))
 (segment (start 138.803666 60.97) (end 146.976 69.142334) (width 0.8) (layer "B.Cu") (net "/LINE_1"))
 (segment (start 136.656 59.27) (end 138.356 60.97) (width 0.8) (layer "B.Cu") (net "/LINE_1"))
 (segment (start 117.636 59.27) (end 119.336 60.97) (width 0.8) (layer "B.Cu") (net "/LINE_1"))
 (segment (start 133.776 94.58) (end 136.35 94.58) (width 0.8) (layer "B.Cu") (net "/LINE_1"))
 (segment (start 100.246 60.97) (end 101.946 59.27) (width 0.8) (layer "B.Cu") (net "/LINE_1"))
 (segment (start 146.976 69.142334) (end 146.976 74.686) (width 0.8) (layer "B.Cu") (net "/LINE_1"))
 (segment (start 119.336 60.97) (end 121.036 59.27) (width 0.8) (layer "B.Cu") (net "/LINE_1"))
 (segment (start 121.036 59.27) (end 136.656 59.27) (width 0.8) (layer "B.Cu") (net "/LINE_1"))
 (segment (start 146.976 74.686) (end 150.57 78.28) (width 0.8) (layer "B.Cu") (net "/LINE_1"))
 (segment (start 136.35 94.58) (end 138.17 96.4) (width 0.8) (layer "B.Cu") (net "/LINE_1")))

